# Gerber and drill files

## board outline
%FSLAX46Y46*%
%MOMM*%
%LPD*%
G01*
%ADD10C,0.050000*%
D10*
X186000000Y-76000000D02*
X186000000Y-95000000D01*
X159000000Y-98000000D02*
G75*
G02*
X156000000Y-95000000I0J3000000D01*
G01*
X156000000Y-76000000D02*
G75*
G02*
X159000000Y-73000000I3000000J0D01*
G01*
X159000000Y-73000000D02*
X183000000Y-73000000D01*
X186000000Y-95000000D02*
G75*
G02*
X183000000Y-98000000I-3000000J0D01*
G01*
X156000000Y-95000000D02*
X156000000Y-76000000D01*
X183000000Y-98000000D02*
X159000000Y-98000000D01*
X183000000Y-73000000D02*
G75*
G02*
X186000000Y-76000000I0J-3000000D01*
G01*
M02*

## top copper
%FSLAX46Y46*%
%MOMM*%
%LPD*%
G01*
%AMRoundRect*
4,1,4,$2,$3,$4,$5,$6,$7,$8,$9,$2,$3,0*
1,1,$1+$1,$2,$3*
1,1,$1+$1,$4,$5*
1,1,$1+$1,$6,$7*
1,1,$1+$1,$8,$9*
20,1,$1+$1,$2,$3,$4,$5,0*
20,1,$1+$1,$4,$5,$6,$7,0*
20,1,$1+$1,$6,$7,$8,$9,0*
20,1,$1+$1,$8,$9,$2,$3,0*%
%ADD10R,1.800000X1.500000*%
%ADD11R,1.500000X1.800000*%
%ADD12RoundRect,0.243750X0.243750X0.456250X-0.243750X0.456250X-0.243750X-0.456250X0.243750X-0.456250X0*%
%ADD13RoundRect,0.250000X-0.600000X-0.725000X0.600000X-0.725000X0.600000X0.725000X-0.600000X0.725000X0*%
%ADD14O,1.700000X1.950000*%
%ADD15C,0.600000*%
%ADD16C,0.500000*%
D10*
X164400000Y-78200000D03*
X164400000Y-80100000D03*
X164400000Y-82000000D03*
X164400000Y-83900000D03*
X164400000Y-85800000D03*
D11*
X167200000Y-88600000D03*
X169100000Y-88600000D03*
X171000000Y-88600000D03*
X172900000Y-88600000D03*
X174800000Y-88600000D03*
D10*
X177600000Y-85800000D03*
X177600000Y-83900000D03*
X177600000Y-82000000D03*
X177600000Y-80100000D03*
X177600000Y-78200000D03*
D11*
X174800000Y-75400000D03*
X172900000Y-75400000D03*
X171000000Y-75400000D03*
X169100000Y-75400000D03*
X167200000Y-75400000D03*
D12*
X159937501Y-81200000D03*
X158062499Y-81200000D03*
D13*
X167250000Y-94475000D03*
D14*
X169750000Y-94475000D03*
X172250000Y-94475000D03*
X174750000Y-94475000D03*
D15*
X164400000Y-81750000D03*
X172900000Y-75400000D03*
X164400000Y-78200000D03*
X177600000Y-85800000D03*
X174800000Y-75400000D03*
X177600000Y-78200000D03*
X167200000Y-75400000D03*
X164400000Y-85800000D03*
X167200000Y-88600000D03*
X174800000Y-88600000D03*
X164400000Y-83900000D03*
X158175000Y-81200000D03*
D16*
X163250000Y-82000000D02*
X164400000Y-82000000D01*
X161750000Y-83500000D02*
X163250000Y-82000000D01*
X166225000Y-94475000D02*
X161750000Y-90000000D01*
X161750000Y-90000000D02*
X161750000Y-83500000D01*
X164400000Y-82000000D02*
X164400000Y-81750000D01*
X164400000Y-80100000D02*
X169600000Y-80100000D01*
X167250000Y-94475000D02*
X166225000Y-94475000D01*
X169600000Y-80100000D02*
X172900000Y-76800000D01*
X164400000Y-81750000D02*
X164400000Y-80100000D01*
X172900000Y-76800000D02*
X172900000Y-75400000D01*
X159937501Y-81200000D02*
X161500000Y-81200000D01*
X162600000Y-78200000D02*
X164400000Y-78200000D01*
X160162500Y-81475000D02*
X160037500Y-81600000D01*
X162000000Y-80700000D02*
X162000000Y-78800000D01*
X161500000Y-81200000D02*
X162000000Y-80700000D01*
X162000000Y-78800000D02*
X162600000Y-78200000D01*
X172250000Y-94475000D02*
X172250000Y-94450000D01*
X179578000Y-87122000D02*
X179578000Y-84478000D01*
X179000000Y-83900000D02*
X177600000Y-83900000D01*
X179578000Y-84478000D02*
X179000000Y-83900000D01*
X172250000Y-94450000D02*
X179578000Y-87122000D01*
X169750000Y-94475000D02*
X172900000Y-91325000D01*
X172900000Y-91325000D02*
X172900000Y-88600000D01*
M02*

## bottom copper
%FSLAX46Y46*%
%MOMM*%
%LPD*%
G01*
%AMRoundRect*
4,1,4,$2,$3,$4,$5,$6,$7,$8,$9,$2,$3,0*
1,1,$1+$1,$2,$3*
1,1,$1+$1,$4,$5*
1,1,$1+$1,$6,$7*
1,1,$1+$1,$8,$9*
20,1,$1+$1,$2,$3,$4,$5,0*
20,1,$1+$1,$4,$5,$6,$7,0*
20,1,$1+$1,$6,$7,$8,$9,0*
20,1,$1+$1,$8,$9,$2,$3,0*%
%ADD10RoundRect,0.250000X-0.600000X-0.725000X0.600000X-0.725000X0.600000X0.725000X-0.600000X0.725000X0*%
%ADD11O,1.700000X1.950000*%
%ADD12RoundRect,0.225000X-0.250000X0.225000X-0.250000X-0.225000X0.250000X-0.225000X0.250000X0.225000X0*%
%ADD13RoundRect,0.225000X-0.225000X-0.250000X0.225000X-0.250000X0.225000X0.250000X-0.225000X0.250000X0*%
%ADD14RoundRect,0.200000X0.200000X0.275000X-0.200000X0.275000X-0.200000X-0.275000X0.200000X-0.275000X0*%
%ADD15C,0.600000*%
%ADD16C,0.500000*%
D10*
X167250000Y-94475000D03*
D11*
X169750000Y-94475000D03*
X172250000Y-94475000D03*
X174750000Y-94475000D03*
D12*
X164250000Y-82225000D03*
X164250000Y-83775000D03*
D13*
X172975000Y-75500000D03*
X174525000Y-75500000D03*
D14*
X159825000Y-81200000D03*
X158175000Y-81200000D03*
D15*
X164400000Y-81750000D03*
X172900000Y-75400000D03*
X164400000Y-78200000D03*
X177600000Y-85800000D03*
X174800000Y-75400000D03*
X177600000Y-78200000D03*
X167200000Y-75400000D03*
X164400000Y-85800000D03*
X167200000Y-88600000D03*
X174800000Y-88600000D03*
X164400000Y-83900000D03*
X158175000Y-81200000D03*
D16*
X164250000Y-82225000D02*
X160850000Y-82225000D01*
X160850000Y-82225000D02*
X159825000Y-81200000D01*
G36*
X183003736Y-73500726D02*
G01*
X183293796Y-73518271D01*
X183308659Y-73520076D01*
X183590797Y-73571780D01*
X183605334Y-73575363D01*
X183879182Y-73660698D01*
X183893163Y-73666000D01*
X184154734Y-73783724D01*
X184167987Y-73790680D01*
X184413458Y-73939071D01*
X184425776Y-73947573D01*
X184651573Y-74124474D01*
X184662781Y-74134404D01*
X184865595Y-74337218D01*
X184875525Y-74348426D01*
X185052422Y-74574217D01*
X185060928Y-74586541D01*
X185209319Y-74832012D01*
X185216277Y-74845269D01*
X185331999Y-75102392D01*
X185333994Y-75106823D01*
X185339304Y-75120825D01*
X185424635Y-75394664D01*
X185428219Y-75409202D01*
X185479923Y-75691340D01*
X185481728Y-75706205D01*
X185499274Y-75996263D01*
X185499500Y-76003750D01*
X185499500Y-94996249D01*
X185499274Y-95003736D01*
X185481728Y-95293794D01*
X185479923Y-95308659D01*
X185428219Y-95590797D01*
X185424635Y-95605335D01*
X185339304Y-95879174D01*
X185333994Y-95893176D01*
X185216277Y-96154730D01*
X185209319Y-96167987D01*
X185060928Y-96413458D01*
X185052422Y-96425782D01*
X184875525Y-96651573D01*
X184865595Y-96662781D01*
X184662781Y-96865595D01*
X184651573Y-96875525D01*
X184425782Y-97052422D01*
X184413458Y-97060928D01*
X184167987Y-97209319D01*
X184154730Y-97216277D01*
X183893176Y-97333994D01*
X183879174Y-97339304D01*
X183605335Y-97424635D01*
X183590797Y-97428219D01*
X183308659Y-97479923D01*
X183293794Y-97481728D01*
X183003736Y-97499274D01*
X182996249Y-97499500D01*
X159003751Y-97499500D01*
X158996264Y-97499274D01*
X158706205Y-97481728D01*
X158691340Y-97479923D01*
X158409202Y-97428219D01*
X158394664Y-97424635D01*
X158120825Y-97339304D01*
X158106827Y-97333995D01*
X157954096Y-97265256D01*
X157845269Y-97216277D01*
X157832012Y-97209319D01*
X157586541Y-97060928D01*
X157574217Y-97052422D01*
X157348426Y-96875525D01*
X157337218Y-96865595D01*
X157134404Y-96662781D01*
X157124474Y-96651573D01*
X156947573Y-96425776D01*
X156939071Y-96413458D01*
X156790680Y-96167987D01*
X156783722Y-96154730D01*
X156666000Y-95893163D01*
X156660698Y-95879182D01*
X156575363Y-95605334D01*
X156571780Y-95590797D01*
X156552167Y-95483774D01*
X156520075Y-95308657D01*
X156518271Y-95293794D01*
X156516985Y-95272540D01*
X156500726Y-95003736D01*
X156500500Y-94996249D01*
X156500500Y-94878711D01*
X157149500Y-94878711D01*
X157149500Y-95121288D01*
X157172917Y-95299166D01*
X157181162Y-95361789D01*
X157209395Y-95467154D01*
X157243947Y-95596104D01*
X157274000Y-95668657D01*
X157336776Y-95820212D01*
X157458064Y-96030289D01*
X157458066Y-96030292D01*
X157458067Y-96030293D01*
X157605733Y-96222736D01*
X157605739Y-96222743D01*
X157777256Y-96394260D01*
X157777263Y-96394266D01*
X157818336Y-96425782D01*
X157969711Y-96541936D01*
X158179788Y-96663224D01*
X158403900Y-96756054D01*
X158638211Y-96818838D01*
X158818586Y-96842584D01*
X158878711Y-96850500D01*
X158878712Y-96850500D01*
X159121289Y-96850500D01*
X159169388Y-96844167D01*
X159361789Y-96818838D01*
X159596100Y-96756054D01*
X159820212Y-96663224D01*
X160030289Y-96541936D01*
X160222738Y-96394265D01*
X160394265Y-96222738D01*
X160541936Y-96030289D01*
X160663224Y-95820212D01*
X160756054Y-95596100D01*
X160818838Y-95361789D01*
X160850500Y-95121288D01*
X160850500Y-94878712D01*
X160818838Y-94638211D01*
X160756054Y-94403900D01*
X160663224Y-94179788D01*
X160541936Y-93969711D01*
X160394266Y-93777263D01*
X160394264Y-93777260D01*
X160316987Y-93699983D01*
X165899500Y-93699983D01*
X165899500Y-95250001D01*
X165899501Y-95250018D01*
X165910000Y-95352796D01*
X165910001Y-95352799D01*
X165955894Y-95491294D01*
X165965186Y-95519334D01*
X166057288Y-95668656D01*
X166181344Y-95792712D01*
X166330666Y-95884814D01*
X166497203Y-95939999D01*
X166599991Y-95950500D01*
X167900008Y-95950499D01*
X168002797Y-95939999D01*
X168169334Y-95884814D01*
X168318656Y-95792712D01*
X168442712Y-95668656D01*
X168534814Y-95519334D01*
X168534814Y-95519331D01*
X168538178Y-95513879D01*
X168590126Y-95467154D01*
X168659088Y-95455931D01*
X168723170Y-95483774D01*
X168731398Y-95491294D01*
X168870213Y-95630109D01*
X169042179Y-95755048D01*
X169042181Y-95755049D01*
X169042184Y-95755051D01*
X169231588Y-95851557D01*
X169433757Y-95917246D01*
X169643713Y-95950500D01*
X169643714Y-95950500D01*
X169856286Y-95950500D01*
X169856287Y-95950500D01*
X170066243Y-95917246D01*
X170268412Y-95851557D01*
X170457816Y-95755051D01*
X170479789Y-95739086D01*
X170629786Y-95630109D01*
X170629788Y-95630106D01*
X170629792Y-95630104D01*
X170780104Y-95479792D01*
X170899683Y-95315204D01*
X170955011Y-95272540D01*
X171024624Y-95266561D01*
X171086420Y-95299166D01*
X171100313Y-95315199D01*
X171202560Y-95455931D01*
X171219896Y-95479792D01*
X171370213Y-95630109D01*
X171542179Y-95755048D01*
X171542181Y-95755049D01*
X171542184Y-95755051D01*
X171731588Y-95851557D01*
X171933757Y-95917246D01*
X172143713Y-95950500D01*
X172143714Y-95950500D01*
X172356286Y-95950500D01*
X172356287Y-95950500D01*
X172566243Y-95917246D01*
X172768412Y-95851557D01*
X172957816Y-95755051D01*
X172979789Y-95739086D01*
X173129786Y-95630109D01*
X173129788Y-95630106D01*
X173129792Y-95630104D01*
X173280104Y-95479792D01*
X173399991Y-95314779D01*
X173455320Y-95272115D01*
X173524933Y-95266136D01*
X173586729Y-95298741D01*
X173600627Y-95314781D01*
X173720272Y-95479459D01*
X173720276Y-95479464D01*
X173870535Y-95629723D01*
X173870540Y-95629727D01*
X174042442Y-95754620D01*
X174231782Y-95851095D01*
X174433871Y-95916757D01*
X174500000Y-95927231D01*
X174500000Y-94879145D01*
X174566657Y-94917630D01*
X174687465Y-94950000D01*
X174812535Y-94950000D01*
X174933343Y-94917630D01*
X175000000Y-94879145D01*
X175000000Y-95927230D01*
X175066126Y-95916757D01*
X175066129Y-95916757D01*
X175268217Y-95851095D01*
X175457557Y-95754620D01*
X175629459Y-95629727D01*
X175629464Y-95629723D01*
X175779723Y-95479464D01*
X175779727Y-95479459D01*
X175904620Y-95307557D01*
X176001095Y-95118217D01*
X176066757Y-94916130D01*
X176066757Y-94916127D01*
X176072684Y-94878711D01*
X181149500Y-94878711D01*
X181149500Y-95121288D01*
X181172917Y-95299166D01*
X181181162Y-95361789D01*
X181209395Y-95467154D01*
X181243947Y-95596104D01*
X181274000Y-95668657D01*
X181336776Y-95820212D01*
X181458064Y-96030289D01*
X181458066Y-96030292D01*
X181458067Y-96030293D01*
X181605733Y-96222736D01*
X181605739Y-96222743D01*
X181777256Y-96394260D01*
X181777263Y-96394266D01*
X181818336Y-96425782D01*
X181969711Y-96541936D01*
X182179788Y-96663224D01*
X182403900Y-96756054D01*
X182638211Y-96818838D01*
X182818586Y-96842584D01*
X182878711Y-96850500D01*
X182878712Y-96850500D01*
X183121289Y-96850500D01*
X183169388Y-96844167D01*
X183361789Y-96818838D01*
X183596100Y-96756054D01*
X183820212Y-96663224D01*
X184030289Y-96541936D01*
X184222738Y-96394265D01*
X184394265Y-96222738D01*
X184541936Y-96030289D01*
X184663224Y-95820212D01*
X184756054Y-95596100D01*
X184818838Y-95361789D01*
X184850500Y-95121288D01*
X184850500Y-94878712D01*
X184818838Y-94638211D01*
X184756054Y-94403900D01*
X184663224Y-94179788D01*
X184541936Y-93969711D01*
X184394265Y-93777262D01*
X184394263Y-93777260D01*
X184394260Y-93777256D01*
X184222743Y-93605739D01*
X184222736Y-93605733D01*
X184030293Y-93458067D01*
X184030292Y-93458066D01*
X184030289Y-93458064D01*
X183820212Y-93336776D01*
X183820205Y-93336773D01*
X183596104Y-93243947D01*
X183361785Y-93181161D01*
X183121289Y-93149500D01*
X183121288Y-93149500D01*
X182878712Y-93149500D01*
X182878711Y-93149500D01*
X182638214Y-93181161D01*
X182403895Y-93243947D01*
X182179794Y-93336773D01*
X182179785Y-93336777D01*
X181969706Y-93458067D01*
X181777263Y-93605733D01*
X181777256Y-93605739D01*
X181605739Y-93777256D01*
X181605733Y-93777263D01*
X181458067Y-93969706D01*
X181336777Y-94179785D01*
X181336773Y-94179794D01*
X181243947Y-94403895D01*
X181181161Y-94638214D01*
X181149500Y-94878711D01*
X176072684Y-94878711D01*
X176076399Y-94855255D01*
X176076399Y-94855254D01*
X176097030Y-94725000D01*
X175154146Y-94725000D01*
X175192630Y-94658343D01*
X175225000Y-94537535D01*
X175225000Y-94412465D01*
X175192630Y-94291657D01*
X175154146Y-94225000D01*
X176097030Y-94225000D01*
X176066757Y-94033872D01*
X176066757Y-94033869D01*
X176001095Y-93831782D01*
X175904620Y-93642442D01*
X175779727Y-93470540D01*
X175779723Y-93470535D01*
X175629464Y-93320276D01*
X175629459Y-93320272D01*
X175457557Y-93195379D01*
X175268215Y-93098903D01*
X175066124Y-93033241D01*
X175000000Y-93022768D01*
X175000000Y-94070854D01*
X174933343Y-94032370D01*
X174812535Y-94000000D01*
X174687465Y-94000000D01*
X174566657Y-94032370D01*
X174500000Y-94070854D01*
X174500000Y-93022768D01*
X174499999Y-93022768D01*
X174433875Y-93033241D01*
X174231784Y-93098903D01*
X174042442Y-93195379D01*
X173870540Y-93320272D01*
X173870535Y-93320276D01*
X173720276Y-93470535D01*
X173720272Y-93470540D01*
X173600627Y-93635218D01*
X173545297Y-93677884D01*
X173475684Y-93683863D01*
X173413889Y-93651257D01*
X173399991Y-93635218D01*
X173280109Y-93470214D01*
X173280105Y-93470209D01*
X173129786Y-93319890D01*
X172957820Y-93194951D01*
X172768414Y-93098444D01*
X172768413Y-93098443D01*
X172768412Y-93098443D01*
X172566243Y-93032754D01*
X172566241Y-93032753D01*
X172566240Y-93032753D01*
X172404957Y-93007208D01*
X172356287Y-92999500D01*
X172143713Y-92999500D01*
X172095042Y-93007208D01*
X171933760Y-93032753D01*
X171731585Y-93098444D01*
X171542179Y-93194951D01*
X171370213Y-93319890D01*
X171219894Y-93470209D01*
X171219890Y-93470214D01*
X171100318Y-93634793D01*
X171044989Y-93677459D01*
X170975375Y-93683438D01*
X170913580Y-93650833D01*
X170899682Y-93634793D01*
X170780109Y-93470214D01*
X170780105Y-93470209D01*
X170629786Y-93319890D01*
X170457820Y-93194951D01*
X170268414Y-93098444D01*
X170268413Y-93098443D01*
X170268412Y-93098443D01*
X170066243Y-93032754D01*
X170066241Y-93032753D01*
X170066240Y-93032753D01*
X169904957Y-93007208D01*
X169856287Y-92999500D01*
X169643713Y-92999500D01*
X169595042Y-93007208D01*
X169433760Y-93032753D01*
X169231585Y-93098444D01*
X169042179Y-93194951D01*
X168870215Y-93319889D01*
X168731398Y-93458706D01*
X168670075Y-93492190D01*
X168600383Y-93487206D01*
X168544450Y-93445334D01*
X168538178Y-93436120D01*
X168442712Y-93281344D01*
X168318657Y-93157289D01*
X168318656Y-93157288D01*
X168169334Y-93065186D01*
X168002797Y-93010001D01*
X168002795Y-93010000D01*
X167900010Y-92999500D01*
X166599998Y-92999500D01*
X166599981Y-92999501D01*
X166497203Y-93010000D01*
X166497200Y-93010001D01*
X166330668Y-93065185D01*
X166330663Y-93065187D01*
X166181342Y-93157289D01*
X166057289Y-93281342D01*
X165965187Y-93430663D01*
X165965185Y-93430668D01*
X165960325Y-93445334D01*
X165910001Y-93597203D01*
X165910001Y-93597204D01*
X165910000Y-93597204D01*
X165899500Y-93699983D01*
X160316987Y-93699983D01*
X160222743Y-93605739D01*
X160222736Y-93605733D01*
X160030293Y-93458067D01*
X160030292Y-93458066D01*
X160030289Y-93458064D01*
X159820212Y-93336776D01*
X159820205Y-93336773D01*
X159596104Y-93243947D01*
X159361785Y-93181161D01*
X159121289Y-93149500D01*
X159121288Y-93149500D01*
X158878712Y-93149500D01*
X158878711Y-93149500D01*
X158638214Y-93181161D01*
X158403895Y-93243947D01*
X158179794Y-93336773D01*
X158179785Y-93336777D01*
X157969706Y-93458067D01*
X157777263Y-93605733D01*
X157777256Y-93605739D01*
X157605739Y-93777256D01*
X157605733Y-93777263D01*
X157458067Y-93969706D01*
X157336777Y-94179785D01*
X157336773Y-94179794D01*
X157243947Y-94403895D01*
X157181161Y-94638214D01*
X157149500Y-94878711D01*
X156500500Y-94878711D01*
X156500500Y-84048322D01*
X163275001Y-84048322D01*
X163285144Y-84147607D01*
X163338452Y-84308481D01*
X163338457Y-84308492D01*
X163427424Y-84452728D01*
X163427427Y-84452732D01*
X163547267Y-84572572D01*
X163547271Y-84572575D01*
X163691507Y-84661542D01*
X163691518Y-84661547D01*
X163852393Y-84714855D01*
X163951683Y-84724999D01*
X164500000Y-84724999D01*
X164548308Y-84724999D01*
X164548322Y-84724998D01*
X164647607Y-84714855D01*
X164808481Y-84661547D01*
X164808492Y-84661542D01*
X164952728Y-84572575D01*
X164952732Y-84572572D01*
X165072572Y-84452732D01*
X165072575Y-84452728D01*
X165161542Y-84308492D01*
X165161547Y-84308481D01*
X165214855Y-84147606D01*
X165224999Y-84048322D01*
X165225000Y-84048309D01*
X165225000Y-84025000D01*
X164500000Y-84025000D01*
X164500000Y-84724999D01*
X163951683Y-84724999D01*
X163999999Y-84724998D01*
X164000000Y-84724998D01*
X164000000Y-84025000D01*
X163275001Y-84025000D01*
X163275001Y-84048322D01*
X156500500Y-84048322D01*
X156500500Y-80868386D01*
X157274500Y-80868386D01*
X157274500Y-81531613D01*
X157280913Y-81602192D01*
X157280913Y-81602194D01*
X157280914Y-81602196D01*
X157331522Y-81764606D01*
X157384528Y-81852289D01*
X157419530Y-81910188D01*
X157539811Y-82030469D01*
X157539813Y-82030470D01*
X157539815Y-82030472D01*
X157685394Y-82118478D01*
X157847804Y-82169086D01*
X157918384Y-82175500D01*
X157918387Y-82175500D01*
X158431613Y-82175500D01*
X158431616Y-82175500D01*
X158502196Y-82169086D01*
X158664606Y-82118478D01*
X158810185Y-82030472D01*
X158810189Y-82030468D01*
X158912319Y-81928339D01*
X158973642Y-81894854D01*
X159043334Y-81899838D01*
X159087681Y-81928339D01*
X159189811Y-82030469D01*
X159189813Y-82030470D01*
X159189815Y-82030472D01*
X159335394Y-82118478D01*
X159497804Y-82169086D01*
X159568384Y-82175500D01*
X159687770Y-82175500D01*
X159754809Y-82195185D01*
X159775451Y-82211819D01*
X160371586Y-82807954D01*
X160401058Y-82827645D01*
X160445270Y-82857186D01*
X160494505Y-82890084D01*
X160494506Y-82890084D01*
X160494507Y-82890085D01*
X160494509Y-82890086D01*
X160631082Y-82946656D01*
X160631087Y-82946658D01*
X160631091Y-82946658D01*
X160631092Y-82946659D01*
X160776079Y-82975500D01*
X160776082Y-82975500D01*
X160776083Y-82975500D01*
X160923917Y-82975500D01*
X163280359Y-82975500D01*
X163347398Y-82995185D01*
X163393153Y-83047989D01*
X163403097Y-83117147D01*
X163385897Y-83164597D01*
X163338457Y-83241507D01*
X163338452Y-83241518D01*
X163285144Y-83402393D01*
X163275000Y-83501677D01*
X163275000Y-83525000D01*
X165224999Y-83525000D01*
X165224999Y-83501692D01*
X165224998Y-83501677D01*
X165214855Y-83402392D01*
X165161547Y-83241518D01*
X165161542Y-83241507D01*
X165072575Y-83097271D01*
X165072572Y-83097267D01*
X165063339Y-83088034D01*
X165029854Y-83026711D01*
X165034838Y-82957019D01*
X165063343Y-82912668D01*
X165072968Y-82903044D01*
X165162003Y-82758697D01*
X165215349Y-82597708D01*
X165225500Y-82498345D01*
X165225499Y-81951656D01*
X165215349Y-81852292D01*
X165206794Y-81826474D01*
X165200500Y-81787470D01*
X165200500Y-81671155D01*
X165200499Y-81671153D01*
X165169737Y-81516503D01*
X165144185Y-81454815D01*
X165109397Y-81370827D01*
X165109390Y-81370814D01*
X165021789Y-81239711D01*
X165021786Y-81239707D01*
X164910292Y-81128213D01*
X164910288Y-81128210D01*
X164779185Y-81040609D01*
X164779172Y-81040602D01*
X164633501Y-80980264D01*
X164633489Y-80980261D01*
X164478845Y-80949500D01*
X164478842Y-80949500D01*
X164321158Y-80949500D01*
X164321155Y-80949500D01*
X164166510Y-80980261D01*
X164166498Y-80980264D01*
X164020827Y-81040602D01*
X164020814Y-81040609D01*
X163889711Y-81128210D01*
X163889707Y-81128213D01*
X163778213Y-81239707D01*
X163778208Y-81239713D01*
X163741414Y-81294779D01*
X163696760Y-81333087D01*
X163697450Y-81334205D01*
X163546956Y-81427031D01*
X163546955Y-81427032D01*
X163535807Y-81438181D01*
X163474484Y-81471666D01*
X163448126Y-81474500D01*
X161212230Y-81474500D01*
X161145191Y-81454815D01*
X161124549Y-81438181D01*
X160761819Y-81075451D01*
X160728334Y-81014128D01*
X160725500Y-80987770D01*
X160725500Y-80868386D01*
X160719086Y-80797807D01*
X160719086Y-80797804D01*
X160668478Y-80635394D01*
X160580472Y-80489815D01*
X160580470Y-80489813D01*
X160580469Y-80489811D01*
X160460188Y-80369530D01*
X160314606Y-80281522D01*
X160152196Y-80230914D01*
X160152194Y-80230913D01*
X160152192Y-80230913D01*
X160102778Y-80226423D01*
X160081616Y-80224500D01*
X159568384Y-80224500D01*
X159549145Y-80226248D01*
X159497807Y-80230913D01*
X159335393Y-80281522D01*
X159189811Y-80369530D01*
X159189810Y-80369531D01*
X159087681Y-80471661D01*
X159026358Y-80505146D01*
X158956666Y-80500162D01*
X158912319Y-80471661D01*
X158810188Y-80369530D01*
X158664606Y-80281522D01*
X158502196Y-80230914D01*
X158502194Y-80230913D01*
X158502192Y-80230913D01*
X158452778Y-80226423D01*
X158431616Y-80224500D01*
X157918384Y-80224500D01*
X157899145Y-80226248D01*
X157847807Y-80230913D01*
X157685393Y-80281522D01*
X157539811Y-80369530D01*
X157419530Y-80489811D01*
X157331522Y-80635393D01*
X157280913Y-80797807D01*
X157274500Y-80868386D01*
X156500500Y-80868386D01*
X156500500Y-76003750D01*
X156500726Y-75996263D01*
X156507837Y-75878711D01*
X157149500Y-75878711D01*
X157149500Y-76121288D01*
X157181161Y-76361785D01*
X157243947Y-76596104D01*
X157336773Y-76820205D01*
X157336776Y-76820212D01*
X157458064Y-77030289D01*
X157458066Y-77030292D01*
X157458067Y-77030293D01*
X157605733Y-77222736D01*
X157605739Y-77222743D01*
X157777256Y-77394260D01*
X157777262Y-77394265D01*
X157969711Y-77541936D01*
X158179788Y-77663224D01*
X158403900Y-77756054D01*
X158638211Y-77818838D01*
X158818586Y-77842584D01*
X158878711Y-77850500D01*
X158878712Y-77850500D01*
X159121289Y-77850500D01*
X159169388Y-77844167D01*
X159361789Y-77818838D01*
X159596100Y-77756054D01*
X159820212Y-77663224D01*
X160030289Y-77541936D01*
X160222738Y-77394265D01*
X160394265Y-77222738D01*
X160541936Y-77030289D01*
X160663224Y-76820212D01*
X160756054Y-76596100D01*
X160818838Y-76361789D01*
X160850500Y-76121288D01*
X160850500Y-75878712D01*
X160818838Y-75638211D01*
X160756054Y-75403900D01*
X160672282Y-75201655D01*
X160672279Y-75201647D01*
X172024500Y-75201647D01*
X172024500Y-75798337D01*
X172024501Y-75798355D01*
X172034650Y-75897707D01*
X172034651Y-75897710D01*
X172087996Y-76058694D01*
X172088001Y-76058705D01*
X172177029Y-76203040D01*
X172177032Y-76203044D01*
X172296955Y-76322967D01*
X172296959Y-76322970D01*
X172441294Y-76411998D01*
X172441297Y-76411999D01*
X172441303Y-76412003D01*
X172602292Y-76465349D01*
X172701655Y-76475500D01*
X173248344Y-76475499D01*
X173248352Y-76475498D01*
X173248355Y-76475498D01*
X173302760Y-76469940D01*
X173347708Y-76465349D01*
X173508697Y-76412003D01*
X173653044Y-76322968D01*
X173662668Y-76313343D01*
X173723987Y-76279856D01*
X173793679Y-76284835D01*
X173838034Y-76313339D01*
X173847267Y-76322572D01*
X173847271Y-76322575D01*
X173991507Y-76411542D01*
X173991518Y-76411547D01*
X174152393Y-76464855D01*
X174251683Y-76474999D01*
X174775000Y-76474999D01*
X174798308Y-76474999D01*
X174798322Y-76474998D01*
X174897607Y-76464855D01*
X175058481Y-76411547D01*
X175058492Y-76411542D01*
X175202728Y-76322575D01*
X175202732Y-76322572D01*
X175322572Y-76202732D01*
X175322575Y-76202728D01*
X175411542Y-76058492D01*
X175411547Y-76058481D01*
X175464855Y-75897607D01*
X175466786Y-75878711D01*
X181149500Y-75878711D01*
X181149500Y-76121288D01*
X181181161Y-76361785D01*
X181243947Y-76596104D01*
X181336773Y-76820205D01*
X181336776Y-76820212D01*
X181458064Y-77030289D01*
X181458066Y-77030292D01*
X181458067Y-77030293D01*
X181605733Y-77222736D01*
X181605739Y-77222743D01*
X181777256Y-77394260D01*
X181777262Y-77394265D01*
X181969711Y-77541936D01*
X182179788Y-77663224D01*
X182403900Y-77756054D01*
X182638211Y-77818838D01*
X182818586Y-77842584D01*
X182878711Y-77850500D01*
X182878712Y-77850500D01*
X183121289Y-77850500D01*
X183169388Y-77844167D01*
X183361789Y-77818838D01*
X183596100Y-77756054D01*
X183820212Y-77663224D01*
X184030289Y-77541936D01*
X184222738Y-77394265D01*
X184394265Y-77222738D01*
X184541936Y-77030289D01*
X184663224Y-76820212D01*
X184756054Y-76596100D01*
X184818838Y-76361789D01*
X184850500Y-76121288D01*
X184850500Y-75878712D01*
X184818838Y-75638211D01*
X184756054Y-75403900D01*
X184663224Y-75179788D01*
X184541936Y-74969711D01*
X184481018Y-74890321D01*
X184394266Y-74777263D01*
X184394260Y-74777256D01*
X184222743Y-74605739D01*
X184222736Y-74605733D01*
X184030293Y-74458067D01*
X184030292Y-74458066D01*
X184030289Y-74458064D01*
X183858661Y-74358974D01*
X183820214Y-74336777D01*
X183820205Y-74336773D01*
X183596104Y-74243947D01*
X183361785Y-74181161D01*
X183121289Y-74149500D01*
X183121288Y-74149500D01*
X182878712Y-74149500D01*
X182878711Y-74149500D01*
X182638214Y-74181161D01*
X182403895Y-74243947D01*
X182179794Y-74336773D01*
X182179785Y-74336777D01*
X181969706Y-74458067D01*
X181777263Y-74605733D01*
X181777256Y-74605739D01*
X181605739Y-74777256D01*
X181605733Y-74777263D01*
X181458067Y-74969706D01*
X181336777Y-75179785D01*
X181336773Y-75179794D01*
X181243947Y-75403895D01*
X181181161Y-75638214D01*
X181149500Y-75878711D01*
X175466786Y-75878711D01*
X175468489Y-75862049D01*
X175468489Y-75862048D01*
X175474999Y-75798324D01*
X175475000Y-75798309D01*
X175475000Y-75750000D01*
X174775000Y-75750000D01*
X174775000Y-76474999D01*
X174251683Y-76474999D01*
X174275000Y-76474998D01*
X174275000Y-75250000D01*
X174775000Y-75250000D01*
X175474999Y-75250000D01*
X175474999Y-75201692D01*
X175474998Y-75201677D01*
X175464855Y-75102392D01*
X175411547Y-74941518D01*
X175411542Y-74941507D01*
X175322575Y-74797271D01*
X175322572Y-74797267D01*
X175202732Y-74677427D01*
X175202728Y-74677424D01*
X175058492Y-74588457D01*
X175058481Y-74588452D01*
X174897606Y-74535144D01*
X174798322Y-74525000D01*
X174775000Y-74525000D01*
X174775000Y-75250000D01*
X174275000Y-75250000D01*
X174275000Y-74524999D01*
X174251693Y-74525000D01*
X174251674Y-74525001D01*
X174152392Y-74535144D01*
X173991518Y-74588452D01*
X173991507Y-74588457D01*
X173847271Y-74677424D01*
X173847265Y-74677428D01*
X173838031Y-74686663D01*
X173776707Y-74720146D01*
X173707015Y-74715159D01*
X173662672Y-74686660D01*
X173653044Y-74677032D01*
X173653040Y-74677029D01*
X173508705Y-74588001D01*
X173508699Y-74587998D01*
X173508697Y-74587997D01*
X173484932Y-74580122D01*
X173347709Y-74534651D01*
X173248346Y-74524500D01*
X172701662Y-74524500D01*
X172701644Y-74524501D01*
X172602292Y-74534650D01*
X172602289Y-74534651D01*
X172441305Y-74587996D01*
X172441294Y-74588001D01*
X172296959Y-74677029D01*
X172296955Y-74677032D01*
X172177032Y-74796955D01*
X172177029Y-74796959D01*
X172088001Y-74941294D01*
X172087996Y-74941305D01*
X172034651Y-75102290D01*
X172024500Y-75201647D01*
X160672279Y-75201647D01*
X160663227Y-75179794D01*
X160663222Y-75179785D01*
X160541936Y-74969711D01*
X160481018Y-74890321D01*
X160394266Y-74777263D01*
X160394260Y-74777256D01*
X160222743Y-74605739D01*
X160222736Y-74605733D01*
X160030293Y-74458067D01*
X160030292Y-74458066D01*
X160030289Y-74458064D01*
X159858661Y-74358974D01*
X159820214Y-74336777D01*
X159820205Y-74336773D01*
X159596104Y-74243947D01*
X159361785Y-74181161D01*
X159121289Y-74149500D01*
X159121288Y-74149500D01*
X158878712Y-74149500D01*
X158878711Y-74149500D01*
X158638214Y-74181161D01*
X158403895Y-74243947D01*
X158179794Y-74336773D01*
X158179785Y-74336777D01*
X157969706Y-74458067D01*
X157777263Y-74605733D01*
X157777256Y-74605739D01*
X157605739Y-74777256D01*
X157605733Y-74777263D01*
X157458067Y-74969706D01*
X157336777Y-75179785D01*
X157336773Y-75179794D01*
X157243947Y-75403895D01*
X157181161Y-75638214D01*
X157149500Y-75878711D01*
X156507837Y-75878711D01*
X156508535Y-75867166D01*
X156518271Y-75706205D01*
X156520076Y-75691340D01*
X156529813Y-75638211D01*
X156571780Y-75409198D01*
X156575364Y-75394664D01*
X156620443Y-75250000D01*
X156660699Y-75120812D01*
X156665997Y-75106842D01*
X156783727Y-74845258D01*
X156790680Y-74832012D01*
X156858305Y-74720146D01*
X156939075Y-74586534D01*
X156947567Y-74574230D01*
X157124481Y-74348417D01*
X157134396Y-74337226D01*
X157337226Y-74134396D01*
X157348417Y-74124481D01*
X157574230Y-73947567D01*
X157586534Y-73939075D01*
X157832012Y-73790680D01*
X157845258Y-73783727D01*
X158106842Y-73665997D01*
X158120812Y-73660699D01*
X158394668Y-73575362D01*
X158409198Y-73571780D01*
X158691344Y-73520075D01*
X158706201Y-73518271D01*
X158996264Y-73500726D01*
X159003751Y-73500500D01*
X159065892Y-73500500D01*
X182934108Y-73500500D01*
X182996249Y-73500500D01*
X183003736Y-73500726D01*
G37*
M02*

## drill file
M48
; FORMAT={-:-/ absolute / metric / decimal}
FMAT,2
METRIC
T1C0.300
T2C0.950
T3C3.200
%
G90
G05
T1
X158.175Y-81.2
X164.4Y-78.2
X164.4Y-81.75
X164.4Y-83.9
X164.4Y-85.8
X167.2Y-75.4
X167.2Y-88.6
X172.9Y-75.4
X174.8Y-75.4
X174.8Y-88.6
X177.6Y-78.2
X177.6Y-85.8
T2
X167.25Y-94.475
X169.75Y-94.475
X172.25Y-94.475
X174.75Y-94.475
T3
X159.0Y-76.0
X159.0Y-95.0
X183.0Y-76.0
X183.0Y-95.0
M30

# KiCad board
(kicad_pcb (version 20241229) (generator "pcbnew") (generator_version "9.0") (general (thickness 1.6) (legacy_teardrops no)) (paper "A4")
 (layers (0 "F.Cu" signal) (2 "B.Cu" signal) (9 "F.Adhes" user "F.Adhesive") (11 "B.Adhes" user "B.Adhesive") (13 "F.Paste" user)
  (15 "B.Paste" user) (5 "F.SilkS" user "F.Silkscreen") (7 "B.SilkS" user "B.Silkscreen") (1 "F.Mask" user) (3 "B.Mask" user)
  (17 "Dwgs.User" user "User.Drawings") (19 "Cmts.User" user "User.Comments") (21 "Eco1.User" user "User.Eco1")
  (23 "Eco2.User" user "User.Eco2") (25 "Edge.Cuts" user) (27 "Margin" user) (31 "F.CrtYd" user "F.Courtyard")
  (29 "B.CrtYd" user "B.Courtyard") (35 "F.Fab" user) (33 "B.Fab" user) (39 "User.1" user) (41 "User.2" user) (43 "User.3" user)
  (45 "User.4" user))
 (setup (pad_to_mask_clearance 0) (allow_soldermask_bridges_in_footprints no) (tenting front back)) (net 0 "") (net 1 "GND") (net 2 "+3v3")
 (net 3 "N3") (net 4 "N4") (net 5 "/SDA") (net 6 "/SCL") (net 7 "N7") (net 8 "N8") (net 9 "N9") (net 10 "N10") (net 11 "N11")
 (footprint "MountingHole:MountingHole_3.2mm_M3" (layer "F.Cu") (at 183 76)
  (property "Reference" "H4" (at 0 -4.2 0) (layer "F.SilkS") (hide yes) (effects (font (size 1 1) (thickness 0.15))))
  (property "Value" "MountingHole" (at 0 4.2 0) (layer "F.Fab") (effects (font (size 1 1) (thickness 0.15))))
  (pad "" np_thru_hole circle (at 0 0) (size 3.2 3.2) (drill 3.2) (layers "*.Cu" "*.Mask")))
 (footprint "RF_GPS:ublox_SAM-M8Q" (layer "F.Cu") (at 171 82)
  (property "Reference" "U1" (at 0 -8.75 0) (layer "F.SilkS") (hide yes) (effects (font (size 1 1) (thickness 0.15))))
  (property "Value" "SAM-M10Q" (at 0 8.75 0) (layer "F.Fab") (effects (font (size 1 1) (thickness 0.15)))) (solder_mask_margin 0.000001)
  (pad "" smd rect (at -7.1 -4.225) (size 0.72 0.58) (layers "F.Paste"))
  (pad "" smd rect (at -7.1 -3.375) (size 0.72 0.58) (layers "F.Paste"))
  (pad "" smd rect (at -7.1 -2.325) (size 0.72 0.58) (layers "F.Paste"))
  (pad "" smd rect (at -7.1 -1.475) (size 0.72 0.58) (layers "F.Paste"))
  (pad "" smd rect (at -7.1 -0.425) (size 0.72 0.58) (layers "F.Paste"))
  (pad "" smd rect (at -7.1 0.425) (size 0.72 0.58) (layers "F.Paste"))
  (pad "" smd rect (at -7.1 1.475) (size 0.72 0.58) (layers "F.Paste"))
  (pad "" smd rect (at -7.1 2.325) (size 0.72 0.58) (layers "F.Paste"))
  (pad "" smd rect (at -7.1 3.375) (size 0.72 0.58) (layers "F.Paste"))
  (pad "" smd rect (at -7.1 4.225) (size 0.72 0.58) (layers "F.Paste"))
  (pad "" smd rect (at -6.1 -4.225) (size 0.72 0.58) (layers "F.Paste"))
  (pad "" smd rect (at -6.1 -3.375) (size 0.72 0.58) (layers "F.Paste"))
  (pad "" smd rect (at -6.1 -2.325) (size 0.72 0.58) (layers "F.Paste"))
  (pad "" smd rect (at -6.1 -1.475) (size 0.72 0.58) (layers "F.Paste"))
  (pad "" smd rect (at -6.1 -0.425) (size 0.72 0.58) (layers "F.Paste"))
  (pad "" smd rect (at -6.1 0.425) (size 0.72 0.58) (layers "F.Paste"))
  (pad "" smd rect (at -6.1 1.475) (size 0.72 0.58) (layers "F.Paste"))
  (pad "" smd rect (at -6.1 2.325) (size 0.72 0.58) (layers "F.Paste"))
  (pad "" smd rect (at -6.1 3.375) (size 0.72 0.58) (layers "F.Paste"))
  (pad "" smd rect (at -6.1 4.225) (size 0.72 0.58) (layers "F.Paste"))
  (pad "" smd rect (at -4.225 -7.1) (size 0.58 0.72) (layers "F.Paste"))
  (pad "" smd rect (at -4.225 -6.1) (size 0.58 0.72) (layers "F.Paste"))
  (pad "" smd rect (at -4.225 6.1) (size 0.58 0.72) (layers "F.Paste"))
  (pad "" smd rect (at -4.225 7.1) (size 0.58 0.72) (layers "F.Paste"))
  (pad "" smd rect (at -3.375 -7.1) (size 0.58 0.72) (layers "F.Paste"))
  (pad "" smd rect (at -3.375 -6.1) (size 0.58 0.72) (layers "F.Paste"))
  (pad "" smd rect (at -3.375 6.1) (size 0.58 0.72) (layers "F.Paste"))
  (pad "" smd rect (at -3.375 7.1) (size 0.58 0.72) (layers "F.Paste"))
  (pad "" smd rect (at -2.325 -7.1) (size 0.58 0.72) (layers "F.Paste"))
  (pad "" smd rect (at -2.325 -6.1) (size 0.58 0.72) (layers "F.Paste"))
  (pad "" smd rect (at -2.325 6.1) (size 0.58 0.72) (layers "F.Paste"))
  (pad "" smd rect (at -2.325 7.1) (size 0.58 0.72) (layers "F.Paste"))
  (pad "" smd rect (at -1.475 -7.1) (size 0.58 0.72) (layers "F.Paste"))
  (pad "" smd rect (at -1.475 -6.1) (size 0.58 0.72) (layers "F.Paste"))
  (pad "" smd rect (at -1.475 6.1) (size 0.58 0.72) (layers "F.Paste"))
  (pad "" smd rect (at -1.475 7.1) (size 0.58 0.72) (layers "F.Paste"))
  (pad "" smd rect (at -0.425 -7.1) (size 0.58 0.72) (layers "F.Paste"))
  (pad "" smd rect (at -0.425 -6.1) (size 0.58 0.72) (layers "F.Paste"))
  (pad "" smd rect (at -0.425 6.1) (size 0.58 0.72) (layers "F.Paste"))
  (pad "" smd rect (at -0.425 7.1) (size 0.58 0.72) (layers "F.Paste"))
  (pad "" smd rect (at 0.425 -7.1) (size 0.58 0.72) (layers "F.Paste"))
  (pad "" smd rect (at 0.425 -6.1) (size 0.58 0.72) (layers "F.Paste"))
  (pad "" smd rect (at 0.425 6.1) (size 0.58 0.72) (layers "F.Paste"))
  (pad "" smd rect (at 0.425 7.1) (size 0.58 0.72) (layers "F.Paste"))
  (pad "" smd rect (at 1.475 -7.1) (size 0.58 0.72) (layers "F.Paste"))
  (pad "" smd rect (at 1.475 -6.1) (size 0.58 0.72) (layers "F.Paste"))
  (pad "" smd rect (at 1.475 6.1) (size 0.58 0.72) (layers "F.Paste"))
  (pad "" smd rect (at 1.475 7.1) (size 0.58 0.72) (layers "F.Paste"))
  (pad "" smd rect (at 2.325 -7.1) (size 0.58 0.72) (layers "F.Paste"))
  (pad "" smd rect (at 2.325 -6.1) (size 0.58 0.72) (layers "F.Paste"))
  (pad "" smd rect (at 2.325 6.1) (size 0.58 0.72) (layers "F.Paste"))
  (pad "" smd rect (at 2.325 7.1) (size 0.58 0.72) (layers "F.Paste"))
  (pad "" smd rect (at 3.375 -7.1) (size 0.58 0.72) (layers "F.Paste"))
  (pad "" smd rect (at 3.375 -6.1) (size 0.58 0.72) (layers "F.Paste"))
  (pad "" smd rect (at 3.375 6.1) (size 0.58 0.72) (layers "F.Paste"))
  (pad "" smd rect (at 3.375 7.1) (size 0.58 0.72) (layers "F.Paste"))
  (pad "" smd rect (at 4.225 -7.1) (size 0.58 0.72) (layers "F.Paste"))
  (pad "" smd rect (at 4.225 -6.1) (size 0.58 0.72) (layers "F.Paste"))
  (pad "" smd rect (at 4.225 6.1) (size 0.58 0.72) (layers "F.Paste"))
  (pad "" smd rect (at 4.225 7.1) (size 0.58 0.72) (layers "F.Paste"))
  (pad "" smd rect (at 6.1 -4.225) (size 0.72 0.58) (layers "F.Paste"))
  (pad "" smd rect (at 6.1 -3.375) (size 0.72 0.58) (layers "F.Paste"))
  (pad "" smd rect (at 6.1 -2.325) (size 0.72 0.58) (layers "F.Paste"))
  (pad "" smd rect (at 6.1 -1.475) (size 0.72 0.58) (layers "F.Paste"))
  (pad "" smd rect (at 6.1 -0.425) (size 0.72 0.58) (layers "F.Paste"))
  (pad "" smd rect (at 6.1 0.425) (size 0.72 0.58) (layers "F.Paste"))
  (pad "" smd rect (at 6.1 1.475) (size 0.72 0.58) (layers "F.Paste"))
  (pad "" smd rect (at 6.1 2.325) (size 0.72 0.58) (layers "F.Paste"))
  (pad "" smd rect (at 6.1 3.375) (size 0.72 0.58) (layers "F.Paste"))
  (pad "" smd rect (at 6.1 4.225) (size 0.72 0.58) (layers "F.Paste"))
  (pad "" smd rect (at 7.1 -4.225) (size 0.72 0.58) (layers "F.Paste"))
  (pad "" smd rect (at 7.1 -3.375) (size 0.72 0.58) (layers "F.Paste"))
  (pad "" smd rect (at 7.1 -2.325) (size 0.72 0.58) (layers "F.Paste"))
  (pad "" smd rect (at 7.1 -1.475) (size 0.72 0.58) (layers "F.Paste"))
  (pad "" smd rect (at 7.1 -0.425) (size 0.72 0.58) (layers "F.Paste"))
  (pad "" smd rect (at 7.1 0.425) (size 0.72 0.58) (layers "F.Paste"))
  (pad "" smd rect (at 7.1 1.475) (size 0.72 0.58) (layers "F.Paste"))
  (pad "" smd rect (at 7.1 2.325) (size 0.72 0.58) (layers "F.Paste"))
  (pad "" smd rect (at 7.1 3.375) (size 0.72 0.58) (layers "F.Paste"))
  (pad "" smd rect (at 7.1 4.225) (size 0.72 0.58) (layers "F.Paste"))
  (pad "1" smd rect (at -6.6 -3.8) (size 1.8 1.5) (layers "F.Cu" "F.Mask") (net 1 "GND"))
  (pad "2" smd rect (at -6.6 -1.9) (size 1.8 1.5) (layers "F.Cu" "F.Mask") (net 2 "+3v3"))
  (pad "3" smd rect (at -6.6 0) (size 1.8 1.5) (layers "F.Cu" "F.Mask") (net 2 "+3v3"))
  (pad "4" smd rect (at -6.6 1.9) (size 1.8 1.5) (layers "F.Cu" "F.Mask") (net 1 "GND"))
  (pad "5" smd rect (at -6.6 3.8) (size 1.8 1.5) (layers "F.Cu" "F.Mask") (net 1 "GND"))
  (pad "6" smd rect (at -3.8 6.6) (size 1.5 1.8) (layers "F.Cu" "F.Mask") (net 1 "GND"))
  (pad "7" smd rect (at -1.9 6.6) (size 1.5 1.8) (layers "F.Cu" "F.Mask") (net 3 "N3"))
  (pad "8" smd rect (at 0 6.6) (size 1.5 1.8) (layers "F.Cu" "F.Mask") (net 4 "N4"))
  (pad "9" smd rect (at 1.9 6.6) (size 1.5 1.8) (layers "F.Cu" "F.Mask") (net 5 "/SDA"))
  (pad "10" smd rect (at 3.8 6.6) (size 1.5 1.8) (layers "F.Cu" "F.Mask") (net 1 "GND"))
  (pad "11" smd rect (at 6.6 3.8) (size 1.8 1.5) (layers "F.Cu" "F.Mask") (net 1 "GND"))
  (pad "12" smd rect (at 6.6 1.9) (size 1.8 1.5) (layers "F.Cu" "F.Mask") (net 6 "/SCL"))
  (pad "13" smd rect (at 6.6 0) (size 1.8 1.5) (layers "F.Cu" "F.Mask") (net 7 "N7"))
  (pad "14" smd rect (at 6.6 -1.9) (size 1.8 1.5) (layers "F.Cu" "F.Mask") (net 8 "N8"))
  (pad "15" smd rect (at 6.6 -3.8) (size 1.8 1.5) (layers "F.Cu" "F.Mask") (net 1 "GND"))
  (pad "16" smd rect (at 3.8 -6.6) (size 1.5 1.8) (layers "F.Cu" "F.Mask") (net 1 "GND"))
  (pad "17" smd rect (at 1.9 -6.6) (size 1.5 1.8) (layers "F.Cu" "F.Mask") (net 2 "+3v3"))
  (pad "18" smd rect (at 0 -6.6) (size 1.5 1.8) (layers "F.Cu" "F.Mask") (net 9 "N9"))
  (pad "19" smd rect (at -1.9 -6.6) (size 1.5 1.8) (layers "F.Cu" "F.Mask") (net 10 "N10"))
  (pad "20" smd rect (at -3.8 -6.6) (size 1.5 1.8) (layers "F.Cu" "F.Mask") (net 1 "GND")))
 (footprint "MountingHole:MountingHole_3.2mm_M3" (layer "F.Cu") (at 183 95)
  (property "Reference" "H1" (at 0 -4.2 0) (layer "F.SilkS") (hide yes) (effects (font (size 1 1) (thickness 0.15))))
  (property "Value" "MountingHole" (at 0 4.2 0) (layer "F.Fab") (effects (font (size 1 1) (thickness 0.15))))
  (pad "" np_thru_hole circle (at 0 0) (size 3.2 3.2) (drill 3.2) (layers "*.Cu" "*.Mask")))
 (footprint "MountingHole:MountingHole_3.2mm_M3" (layer "F.Cu") (at 159 76)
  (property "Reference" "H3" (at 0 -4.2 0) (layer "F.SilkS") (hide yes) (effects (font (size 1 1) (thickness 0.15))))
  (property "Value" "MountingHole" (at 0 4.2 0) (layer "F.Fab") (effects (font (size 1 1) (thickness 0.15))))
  (pad "" np_thru_hole circle (at 0 0) (size 3.2 3.2) (drill 3.2) (layers "*.Cu" "*.Mask")))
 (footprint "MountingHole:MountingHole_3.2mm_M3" (layer "F.Cu") (at 159 95)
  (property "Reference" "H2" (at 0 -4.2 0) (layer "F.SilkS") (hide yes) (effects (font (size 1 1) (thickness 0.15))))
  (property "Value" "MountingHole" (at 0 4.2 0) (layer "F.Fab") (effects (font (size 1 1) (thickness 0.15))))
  (pad "" np_thru_hole circle (at 0 0) (size 3.2 3.2) (drill 3.2) (layers "*.Cu" "*.Mask")))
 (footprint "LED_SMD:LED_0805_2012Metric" (layer "F.Cu") (at 159 81.2 180)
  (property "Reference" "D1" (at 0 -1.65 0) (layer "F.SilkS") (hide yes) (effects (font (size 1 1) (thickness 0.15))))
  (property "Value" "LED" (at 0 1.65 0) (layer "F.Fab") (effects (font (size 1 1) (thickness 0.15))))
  (pad "1" smd roundrect (at -0.937501 0 180) (size 0.975 1.4) (layers "F.Cu" "F.Mask" "F.Paste") (roundrect_rratio 0.25) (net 1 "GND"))
  (pad "2" smd roundrect (at 0.937501 0 180) (size 0.975 1.4) (layers "F.Cu" "F.Mask" "F.Paste") (roundrect_rratio 0.25) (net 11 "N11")))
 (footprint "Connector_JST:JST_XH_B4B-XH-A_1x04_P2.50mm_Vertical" (layer "F.Cu") (at 167.25 94.475)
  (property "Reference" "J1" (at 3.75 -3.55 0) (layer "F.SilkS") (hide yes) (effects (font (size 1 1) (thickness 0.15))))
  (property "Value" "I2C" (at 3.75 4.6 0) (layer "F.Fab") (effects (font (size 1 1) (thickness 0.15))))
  (pad "1" thru_hole roundrect (at 0 0) (size 1.7 1.95) (drill 0.95) (layers "*.Cu" "*.Mask") (remove_unused_layers no)
   (roundrect_rratio 0.147059) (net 2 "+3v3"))
  (pad "2" thru_hole oval (at 2.5 0) (size 1.7 1.95) (drill 0.95) (layers "*.Cu" "*.Mask") (remove_unused_layers no) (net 5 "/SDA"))
  (pad "3" thru_hole oval (at 5 0) (size 1.7 1.95) (drill 0.95) (layers "*.Cu" "*.Mask") (remove_unused_layers no) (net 6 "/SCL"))
  (pad "4" thru_hole oval (at 7.5 0) (size 1.7 1.95) (drill 0.95) (layers "*.Cu" "*.Mask") (remove_unused_layers no) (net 1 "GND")))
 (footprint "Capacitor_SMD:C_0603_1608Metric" (layer "B.Cu") (at 164.25 83 -90)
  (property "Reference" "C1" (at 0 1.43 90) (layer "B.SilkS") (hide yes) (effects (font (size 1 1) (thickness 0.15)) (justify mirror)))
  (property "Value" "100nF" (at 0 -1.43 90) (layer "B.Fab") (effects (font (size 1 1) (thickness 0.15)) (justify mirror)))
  (pad "1" smd roundrect (at -0.775 0 270) (size 0.9 0.95) (layers "B.Cu" "B.Mask" "B.Paste") (roundrect_rratio 0.25) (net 2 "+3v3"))
  (pad "2" smd roundrect (at 0.775 0 270) (size 0.9 0.95) (layers "B.Cu" "B.Mask" "B.Paste") (roundrect_rratio 0.25) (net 1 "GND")))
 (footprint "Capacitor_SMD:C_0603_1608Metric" (layer "B.Cu") (at 173.75 75.5)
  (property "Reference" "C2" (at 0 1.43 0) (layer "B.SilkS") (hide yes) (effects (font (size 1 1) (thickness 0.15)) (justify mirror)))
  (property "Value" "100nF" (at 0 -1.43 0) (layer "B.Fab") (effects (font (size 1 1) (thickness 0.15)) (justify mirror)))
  (pad "1" smd roundrect (at -0.775 0) (size 0.9 0.95) (layers "B.Cu" "B.Mask" "B.Paste") (roundrect_rratio 0.25) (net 2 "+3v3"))
  (pad "2" smd roundrect (at 0.775 0) (size 0.9 0.95) (layers "B.Cu" "B.Mask" "B.Paste") (roundrect_rratio 0.25) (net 1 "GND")))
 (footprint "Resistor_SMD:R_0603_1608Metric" (layer "B.Cu") (at 159 81.2 180)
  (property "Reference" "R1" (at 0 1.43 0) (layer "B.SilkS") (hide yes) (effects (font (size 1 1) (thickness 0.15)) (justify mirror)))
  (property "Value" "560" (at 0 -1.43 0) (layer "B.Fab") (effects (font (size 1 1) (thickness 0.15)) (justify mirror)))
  (pad "1" smd roundrect (at -0.825 0 180) (size 0.8 0.95) (layers "B.Cu" "B.Mask" "B.Paste") (roundrect_rratio 0.25) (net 2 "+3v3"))
  (pad "2" smd roundrect (at 0.825 0 180) (size 0.8 0.95) (layers "B.Cu" "B.Mask" "B.Paste") (roundrect_rratio 0.25) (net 11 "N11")))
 (gr_line (start 186 76) (end 186 95) (stroke (width 0.05) (type default)) (layer "Edge.Cuts"))
 (gr_arc (start 159 98) (mid 156.87868 97.12132) (end 156 95) (stroke (width 0.05) (type default)) (layer "Edge.Cuts"))
 (gr_arc (start 156 76) (mid 156.87868 73.87868) (end 159 73) (stroke (width 0.05) (type default)) (layer "Edge.Cuts"))
 (gr_line (start 159 73) (end 183 73) (stroke (width 0.05) (type default)) (layer "Edge.Cuts"))
 (gr_arc (start 186 95) (mid 185.12132 97.12132) (end 183 98) (stroke (width 0.05) (type default)) (layer "Edge.Cuts"))
 (gr_line (start 156 95) (end 156 76) (stroke (width 0.05) (type default)) (layer "Edge.Cuts"))
 (gr_line (start 183 98) (end 159 98) (stroke (width 0.05) (type default)) (layer "Edge.Cuts"))
 (gr_arc (start 183 73) (mid 185.12132 73.87868) (end 186 76) (stroke (width 0.05) (type default)) (layer "Edge.Cuts"))
 (segment (start 163.25 82) (end 164.4 82) (width 0.5) (layer "F.Cu") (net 2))
 (segment (start 161.75 83.5) (end 163.25 82) (width 0.5) (layer "F.Cu") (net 2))
 (segment (start 166.225 94.475) (end 161.75 90) (width 0.5) (layer "F.Cu") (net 2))
 (segment (start 161.75 90) (end 161.75 83.5) (width 0.5) (layer "F.Cu") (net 2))
 (segment (start 164.4 82) (end 164.4 81.75) (width 0.5) (layer "F.Cu") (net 2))
 (segment (start 164.4 80.1) (end 169.6 80.1) (width 0.5) (layer "F.Cu") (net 2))
 (segment (start 167.25 94.475) (end 166.225 94.475) (width 0.5) (layer "F.Cu") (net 2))
 (segment (start 169.6 80.1) (end 172.9 76.8) (width 0.5) (layer "F.Cu") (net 2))
 (segment (start 164.4 81.75) (end 164.4 80.1) (width 0.5) (layer "F.Cu") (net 2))
 (segment (start 172.9 76.8) (end 172.9 75.4) (width 0.5) (layer "F.Cu") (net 2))
 (via (at 164.4 81.75) (size 0.6) (drill 0.3) (layers "F.Cu" "B.Cu") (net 2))
 (via (at 172.9 75.4) (size 0.6) (drill 0.3) (layers "F.Cu" "B.Cu") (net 2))
 (segment (start 164.25 82.225) (end 160.85 82.225) (width 0.5) (layer "B.Cu") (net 2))
 (segment (start 160.85 82.225) (end 159.825 81.2) (width 0.5) (layer "B.Cu") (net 2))
 (segment (start 159.937501 81.2) (end 161.5 81.2) (width 0.5) (layer "F.Cu") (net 1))
 (segment (start 162.6 78.2) (end 164.4 78.2) (width 0.5) (layer "F.Cu") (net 1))
 (segment (start 160.1625 81.475) (end 160.0375 81.6) (width 0.5) (layer "F.Cu") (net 1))
 (segment (start 162 80.7) (end 162 78.8) (width 0.5) (layer "F.Cu") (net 1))
 (segment (start 161.5 81.2) (end 162 80.7) (width 0.5) (layer "F.Cu") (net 1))
 (segment (start 162 78.8) (end 162.6 78.2) (width 0.5) (layer "F.Cu") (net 1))
 (via (at 164.4 78.2) (size 0.6) (drill 0.3) (layers "F.Cu" "B.Cu") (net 1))
 (via (at 177.6 85.8) (size 0.6) (drill 0.3) (layers "F.Cu" "B.Cu") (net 1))
 (via (at 174.8 75.4) (size 0.6) (drill 0.3) (layers "F.Cu" "B.Cu") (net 1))
 (via (at 177.6 78.2) (size 0.6) (drill 0.3) (layers "F.Cu" "B.Cu") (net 1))
 (via (at 167.2 75.4) (size 0.6) (drill 0.3) (layers "F.Cu" "B.Cu") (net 1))
 (via (at 164.4 85.8) (size 0.6) (drill 0.3) (layers "F.Cu" "B.Cu") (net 1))
 (via (at 167.2 88.6) (size 0.6) (drill 0.3) (layers "F.Cu" "B.Cu") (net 1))
 (via (at 174.8 88.6) (size 0.6) (drill 0.3) (layers "F.Cu" "B.Cu") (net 1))
 (via (at 164.4 83.9) (size 0.6) (drill 0.3) (layers "F.Cu" "B.Cu") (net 1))
 (segment (start 172.25 94.475) (end 172.25 94.45) (width 0.5) (layer "F.Cu") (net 6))
 (segment (start 179.578 87.122) (end 179.578 84.478) (width 0.5) (layer "F.Cu") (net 6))
 (segment (start 179 83.9) (end 177.6 83.9) (width 0.5) (layer "F.Cu") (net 6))
 (segment (start 179.578 84.478) (end 179 83.9) (width 0.5) (layer "F.Cu") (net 6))
 (segment (start 172.25 94.45) (end 179.578 87.122) (width 0.5) (layer "F.Cu") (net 6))
 (segment (start 169.75 94.475) (end 172.9 91.325) (width 0.5) (layer "F.Cu") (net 5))
 (segment (start 172.9 91.325) (end 172.9 88.6) (width 0.5) (layer "F.Cu") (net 5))
 (via (at 158.175 81.2) (size 0.6) (drill 0.3) (layers "F.Cu" "B.Cu") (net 11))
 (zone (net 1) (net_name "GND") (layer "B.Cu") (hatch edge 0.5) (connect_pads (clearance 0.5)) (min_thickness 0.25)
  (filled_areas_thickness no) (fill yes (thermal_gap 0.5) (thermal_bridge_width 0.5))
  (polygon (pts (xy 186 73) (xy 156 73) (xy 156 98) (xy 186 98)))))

